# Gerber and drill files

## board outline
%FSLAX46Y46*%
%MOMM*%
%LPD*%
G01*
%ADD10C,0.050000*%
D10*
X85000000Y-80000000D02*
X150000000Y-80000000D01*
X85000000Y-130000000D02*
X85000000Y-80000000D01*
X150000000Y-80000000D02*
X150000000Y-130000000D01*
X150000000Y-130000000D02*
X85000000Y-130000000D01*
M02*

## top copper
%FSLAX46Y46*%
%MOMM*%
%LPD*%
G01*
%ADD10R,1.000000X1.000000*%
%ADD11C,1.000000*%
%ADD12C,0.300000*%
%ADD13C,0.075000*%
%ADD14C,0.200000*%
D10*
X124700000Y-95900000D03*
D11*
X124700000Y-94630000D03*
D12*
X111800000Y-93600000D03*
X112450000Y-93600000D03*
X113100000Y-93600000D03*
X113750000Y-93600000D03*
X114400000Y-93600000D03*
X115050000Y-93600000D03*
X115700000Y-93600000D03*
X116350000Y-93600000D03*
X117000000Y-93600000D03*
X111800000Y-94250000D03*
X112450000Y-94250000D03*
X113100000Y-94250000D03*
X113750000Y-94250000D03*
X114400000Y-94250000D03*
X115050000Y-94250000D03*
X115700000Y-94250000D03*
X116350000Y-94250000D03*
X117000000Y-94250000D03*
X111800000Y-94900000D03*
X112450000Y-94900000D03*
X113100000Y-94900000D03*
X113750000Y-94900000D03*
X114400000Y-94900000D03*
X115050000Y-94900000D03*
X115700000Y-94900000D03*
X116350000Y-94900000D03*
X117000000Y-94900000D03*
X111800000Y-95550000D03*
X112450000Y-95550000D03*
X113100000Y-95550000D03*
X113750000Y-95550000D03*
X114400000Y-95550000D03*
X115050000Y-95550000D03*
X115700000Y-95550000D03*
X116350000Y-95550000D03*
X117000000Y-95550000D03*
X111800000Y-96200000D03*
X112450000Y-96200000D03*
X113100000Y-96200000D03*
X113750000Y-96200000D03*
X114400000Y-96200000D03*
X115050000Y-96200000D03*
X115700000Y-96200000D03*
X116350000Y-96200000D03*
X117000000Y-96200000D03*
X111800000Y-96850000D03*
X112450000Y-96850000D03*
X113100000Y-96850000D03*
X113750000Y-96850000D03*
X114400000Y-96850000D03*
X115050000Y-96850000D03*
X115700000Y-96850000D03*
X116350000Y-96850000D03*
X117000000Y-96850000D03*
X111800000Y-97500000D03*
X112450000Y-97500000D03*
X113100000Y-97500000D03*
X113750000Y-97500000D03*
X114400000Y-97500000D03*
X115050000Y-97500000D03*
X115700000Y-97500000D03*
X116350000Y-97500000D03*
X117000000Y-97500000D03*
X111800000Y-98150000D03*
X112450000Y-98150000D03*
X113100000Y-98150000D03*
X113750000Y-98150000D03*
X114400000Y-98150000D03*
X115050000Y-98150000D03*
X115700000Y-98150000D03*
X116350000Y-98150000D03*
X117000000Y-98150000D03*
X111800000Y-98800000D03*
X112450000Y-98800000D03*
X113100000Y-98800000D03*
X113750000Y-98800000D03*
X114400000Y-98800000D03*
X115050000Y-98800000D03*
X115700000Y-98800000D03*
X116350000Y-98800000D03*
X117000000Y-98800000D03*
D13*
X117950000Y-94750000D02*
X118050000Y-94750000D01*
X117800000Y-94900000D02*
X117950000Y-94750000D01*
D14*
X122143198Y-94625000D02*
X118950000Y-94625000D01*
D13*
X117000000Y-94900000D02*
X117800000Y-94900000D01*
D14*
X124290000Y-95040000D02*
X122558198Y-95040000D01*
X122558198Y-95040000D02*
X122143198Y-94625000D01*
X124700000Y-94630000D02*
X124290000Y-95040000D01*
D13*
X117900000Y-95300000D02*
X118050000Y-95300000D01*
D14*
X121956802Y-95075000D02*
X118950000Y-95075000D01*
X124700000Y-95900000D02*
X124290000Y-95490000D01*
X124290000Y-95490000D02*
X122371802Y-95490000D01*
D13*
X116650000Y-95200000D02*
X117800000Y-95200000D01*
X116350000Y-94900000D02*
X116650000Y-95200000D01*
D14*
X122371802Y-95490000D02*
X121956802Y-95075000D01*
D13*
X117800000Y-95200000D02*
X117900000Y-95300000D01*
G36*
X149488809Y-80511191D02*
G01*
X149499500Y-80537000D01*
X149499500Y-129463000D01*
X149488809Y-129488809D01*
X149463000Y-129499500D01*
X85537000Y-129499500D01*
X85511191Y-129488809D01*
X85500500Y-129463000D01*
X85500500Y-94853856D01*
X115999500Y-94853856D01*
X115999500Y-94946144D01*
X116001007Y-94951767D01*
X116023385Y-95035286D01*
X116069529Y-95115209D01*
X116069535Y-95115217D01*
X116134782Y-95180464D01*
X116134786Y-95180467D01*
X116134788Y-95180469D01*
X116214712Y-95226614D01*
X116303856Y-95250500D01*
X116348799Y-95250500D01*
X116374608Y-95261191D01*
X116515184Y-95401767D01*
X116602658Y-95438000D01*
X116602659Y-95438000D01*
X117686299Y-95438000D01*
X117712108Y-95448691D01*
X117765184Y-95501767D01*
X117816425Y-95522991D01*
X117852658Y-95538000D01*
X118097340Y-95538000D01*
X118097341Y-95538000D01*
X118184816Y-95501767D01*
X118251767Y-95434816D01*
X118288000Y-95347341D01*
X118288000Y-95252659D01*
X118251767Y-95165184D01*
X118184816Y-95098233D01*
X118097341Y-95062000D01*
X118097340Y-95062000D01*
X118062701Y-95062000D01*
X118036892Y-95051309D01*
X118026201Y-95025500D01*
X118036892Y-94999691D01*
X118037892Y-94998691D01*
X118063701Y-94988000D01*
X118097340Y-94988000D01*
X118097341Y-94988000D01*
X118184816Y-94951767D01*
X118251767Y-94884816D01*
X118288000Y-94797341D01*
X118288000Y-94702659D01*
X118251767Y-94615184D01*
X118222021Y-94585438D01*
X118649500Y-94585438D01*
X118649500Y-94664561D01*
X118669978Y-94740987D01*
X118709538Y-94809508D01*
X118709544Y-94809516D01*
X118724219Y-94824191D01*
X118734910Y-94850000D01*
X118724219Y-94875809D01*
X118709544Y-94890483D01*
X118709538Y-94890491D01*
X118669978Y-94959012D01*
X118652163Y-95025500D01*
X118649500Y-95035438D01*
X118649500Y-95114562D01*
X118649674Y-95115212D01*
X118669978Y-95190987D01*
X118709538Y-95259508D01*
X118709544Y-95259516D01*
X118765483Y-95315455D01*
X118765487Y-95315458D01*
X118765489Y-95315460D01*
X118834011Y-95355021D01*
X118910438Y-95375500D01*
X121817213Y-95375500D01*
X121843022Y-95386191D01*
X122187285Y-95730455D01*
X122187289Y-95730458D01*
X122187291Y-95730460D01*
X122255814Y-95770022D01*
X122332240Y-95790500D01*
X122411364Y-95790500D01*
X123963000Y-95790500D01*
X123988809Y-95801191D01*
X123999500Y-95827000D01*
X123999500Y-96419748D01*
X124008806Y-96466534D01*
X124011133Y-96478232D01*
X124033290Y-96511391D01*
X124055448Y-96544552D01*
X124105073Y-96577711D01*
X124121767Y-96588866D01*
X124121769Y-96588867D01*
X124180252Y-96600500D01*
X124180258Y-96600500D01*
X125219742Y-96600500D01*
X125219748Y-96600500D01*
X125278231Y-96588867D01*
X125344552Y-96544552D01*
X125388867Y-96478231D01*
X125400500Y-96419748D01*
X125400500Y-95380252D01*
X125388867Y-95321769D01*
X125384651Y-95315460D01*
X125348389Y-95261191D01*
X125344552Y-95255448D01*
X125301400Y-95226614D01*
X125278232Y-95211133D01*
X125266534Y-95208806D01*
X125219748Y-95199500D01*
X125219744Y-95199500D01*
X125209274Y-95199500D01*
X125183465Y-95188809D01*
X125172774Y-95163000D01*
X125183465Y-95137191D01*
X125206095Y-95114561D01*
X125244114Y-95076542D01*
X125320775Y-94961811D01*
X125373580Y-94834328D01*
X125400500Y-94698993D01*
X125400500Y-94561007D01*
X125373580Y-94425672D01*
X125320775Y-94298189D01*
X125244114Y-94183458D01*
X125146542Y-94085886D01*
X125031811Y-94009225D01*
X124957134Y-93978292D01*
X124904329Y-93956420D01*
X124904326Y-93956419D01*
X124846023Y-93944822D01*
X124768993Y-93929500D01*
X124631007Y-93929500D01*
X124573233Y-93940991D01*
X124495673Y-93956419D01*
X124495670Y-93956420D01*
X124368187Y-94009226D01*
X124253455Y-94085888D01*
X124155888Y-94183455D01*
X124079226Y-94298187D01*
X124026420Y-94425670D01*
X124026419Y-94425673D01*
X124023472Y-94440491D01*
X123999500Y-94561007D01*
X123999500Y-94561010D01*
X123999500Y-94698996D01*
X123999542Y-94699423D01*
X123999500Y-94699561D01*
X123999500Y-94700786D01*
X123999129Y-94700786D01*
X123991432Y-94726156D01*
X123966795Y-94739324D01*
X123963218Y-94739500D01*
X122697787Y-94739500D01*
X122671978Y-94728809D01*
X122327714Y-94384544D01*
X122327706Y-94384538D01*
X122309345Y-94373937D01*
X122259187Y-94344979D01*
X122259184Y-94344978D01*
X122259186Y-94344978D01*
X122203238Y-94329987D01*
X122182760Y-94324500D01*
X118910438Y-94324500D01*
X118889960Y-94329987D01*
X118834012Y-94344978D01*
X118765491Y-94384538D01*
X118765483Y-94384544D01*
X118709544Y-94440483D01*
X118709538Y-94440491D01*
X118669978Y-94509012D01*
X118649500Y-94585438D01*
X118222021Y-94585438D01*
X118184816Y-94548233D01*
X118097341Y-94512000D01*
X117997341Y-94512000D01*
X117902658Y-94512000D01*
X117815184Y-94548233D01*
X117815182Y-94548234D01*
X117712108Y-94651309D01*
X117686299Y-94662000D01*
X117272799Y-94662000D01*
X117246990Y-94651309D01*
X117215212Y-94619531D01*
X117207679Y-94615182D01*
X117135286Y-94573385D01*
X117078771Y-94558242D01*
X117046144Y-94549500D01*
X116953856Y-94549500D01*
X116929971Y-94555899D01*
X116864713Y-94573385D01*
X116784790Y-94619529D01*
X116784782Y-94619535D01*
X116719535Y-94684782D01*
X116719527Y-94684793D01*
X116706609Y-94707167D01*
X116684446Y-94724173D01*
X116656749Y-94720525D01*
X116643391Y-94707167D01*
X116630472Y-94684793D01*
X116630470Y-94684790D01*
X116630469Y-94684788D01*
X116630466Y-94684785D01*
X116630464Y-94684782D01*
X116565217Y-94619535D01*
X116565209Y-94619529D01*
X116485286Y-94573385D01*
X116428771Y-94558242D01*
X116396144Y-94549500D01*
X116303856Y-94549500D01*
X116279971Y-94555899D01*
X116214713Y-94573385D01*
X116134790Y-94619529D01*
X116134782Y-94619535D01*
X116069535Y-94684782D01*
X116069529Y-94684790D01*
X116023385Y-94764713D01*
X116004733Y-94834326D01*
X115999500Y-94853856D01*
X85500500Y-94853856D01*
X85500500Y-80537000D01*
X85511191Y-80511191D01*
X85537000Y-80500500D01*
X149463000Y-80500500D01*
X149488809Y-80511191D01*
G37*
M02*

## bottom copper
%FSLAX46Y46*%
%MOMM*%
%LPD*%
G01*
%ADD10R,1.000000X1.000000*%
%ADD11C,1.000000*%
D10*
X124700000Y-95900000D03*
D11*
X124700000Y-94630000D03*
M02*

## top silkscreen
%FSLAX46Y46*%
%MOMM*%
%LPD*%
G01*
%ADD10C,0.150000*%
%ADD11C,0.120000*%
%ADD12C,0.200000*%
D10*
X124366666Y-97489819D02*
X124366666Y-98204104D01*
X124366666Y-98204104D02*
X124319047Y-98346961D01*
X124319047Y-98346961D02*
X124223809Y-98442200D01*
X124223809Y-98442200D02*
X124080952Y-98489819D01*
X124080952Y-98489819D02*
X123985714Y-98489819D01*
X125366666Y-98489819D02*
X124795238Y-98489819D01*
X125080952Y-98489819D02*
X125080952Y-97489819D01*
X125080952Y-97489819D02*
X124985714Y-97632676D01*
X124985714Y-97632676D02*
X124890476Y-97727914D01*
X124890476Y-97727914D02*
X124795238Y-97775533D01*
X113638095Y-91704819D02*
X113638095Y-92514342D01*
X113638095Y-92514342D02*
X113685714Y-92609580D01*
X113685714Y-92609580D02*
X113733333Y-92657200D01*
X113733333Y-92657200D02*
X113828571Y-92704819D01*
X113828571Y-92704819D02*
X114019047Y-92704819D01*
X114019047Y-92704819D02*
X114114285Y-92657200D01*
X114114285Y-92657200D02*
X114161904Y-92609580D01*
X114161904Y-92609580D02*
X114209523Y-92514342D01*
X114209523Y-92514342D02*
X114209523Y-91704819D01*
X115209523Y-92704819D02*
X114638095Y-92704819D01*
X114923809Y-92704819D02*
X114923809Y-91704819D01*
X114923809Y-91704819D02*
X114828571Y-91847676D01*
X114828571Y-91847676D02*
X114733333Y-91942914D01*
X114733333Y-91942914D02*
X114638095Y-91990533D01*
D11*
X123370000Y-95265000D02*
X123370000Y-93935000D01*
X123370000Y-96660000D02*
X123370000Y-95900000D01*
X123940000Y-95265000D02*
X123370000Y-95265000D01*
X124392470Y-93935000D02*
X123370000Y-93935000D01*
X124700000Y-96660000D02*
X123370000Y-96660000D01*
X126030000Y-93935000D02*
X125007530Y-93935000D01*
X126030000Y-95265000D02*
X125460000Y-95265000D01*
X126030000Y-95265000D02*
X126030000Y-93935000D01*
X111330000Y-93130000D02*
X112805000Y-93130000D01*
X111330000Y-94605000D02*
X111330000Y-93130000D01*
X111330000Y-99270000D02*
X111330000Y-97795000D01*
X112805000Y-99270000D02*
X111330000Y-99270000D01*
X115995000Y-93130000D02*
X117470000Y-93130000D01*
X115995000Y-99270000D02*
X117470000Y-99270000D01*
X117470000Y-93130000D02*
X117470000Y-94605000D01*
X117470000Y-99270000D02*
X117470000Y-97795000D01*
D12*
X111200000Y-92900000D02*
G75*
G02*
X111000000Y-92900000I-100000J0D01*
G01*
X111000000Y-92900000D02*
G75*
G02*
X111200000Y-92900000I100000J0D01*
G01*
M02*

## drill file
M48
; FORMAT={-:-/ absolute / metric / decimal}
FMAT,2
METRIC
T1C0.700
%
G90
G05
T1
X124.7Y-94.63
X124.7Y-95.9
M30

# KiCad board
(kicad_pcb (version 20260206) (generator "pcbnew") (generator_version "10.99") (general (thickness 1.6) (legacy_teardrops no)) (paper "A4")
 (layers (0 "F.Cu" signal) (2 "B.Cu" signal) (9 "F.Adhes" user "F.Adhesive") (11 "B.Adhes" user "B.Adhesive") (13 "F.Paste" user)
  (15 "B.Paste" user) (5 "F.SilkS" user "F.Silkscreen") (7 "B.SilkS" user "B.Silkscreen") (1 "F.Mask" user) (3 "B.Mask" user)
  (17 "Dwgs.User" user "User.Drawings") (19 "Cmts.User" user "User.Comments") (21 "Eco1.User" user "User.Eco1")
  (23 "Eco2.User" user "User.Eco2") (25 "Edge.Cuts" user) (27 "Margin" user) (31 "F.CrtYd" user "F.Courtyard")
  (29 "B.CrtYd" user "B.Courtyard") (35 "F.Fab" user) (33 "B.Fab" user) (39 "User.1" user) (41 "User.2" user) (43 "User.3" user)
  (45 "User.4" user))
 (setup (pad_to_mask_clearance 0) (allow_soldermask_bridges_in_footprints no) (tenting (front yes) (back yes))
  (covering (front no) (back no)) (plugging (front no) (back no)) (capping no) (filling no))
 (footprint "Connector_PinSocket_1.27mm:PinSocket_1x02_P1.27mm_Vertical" (layer "F.Cu") (at 124.7 95.9 180)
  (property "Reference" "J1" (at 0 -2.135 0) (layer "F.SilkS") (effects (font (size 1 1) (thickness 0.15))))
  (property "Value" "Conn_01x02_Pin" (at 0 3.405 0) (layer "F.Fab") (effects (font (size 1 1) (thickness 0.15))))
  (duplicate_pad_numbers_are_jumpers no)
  (fp_line (start 1.33 0.635) (end 1.33 1.965) (stroke (width 0.12) (type solid)) (layer "F.SilkS"))
  (fp_line (start 1.33 -0.76) (end 1.33 0) (stroke (width 0.12) (type solid)) (layer "F.SilkS"))
  (fp_line (start 0.76 0.635) (end 1.33 0.635) (stroke (width 0.12) (type solid)) (layer "F.SilkS"))
  (fp_line (start 0.30753 1.965) (end 1.33 1.965) (stroke (width 0.12) (type solid)) (layer "F.SilkS"))
  (fp_line (start 0 -0.76) (end 1.33 -0.76) (stroke (width 0.12) (type solid)) (layer "F.SilkS"))
  (fp_line (start -1.33 1.965) (end -0.30753 1.965) (stroke (width 0.12) (type solid)) (layer "F.SilkS"))
  (fp_line (start -1.33 0.635) (end -0.76 0.635) (stroke (width 0.12) (type solid)) (layer "F.SilkS"))
  (fp_line (start -1.33 0.635) (end -1.33 1.965) (stroke (width 0.12) (type solid)) (layer "F.SilkS"))
  (pad "1" thru_hole rect (at 0 0 180) (size 1 1) (drill 0.7) (layers "*.Cu" "*.Mask") (remove_unused_layers no) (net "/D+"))
  (pad "2" thru_hole circle (at 0 1.27 180) (size 1 1) (drill 0.7) (layers "*.Cu" "*.Mask") (remove_unused_layers no) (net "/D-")))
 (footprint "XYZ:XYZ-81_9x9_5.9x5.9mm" (layer "F.Cu") (at 114.4 96.2)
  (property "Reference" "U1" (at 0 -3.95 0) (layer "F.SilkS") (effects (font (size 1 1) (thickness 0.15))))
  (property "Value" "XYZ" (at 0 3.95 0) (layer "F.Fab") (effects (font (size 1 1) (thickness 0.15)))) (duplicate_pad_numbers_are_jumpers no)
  (fp_line (start -3.07 -3.07) (end -1.595 -3.07) (stroke (width 0.12) (type default)) (layer "F.SilkS"))
  (fp_line (start -3.07 -1.595) (end -3.07 -3.07) (stroke (width 0.12) (type default)) (layer "F.SilkS"))
  (fp_line (start -3.07 3.07) (end -3.07 1.595) (stroke (width 0.12) (type default)) (layer "F.SilkS"))
  (fp_line (start -1.595 3.07) (end -3.07 3.07) (stroke (width 0.12) (type default)) (layer "F.SilkS"))
  (fp_line (start 1.595 -3.07) (end 3.07 -3.07) (stroke (width 0.12) (type default)) (layer "F.SilkS"))
  (fp_line (start 1.595 3.07) (end 3.07 3.07) (stroke (width 0.12) (type default)) (layer "F.SilkS"))
  (fp_line (start 3.07 -3.07) (end 3.07 -1.595) (stroke (width 0.12) (type default)) (layer "F.SilkS"))
  (fp_line (start 3.07 3.07) (end 3.07 1.595) (stroke (width 0.12) (type default)) (layer "F.SilkS"))
  (fp_circle (center -3.3 -3.3) (end -3.3 -3.2) (stroke (width 0.2) (type default)) (fill no) (layer "F.SilkS"))
  (pad "A1" smd circle (at -2.6 -2.6) (size 0.3 0.3) (layers "F.Cu" "F.Mask" "F.Paste") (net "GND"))
  (pad "A2" smd circle (at -1.95 -2.6) (size 0.3 0.3) (layers "F.Cu" "F.Mask" "F.Paste") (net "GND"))
  (pad "A3" smd circle (at -1.3 -2.6) (size 0.3 0.3) (layers "F.Cu" "F.Mask" "F.Paste") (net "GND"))
  (pad "A4" smd circle (at -0.65 -2.6) (size 0.3 0.3) (layers "F.Cu" "F.Mask" "F.Paste") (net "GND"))
  (pad "A5" smd circle (at 0 -2.6) (size 0.3 0.3) (layers "F.Cu" "F.Mask" "F.Paste") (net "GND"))
  (pad "A6" smd circle (at 0.65 -2.6) (size 0.3 0.3) (layers "F.Cu" "F.Mask" "F.Paste") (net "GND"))
  (pad "A7" smd circle (at 1.3 -2.6) (size 0.3 0.3) (layers "F.Cu" "F.Mask" "F.Paste") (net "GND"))
  (pad "A8" smd circle (at 1.95 -2.6) (size 0.3 0.3) (layers "F.Cu" "F.Mask" "F.Paste") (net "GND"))
  (pad "A9" smd circle (at 2.6 -2.6) (size 0.3 0.3) (layers "F.Cu" "F.Mask" "F.Paste") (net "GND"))
  (pad "B1" smd circle (at -2.6 -1.95) (size 0.3 0.3) (layers "F.Cu" "F.Mask" "F.Paste") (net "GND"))
  (pad "B2" smd circle (at -1.95 -1.95) (size 0.3 0.3) (layers "F.Cu" "F.Mask" "F.Paste") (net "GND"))
  (pad "B3" smd circle (at -1.3 -1.95) (size 0.3 0.3) (layers "F.Cu" "F.Mask" "F.Paste") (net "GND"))
  (pad "B4" smd circle (at -0.65 -1.95) (size 0.3 0.3) (layers "F.Cu" "F.Mask" "F.Paste") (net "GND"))
  (pad "B5" smd circle (at 0 -1.95) (size 0.3 0.3) (layers "F.Cu" "F.Mask" "F.Paste") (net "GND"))
  (pad "B6" smd circle (at 0.65 -1.95) (size 0.3 0.3) (layers "F.Cu" "F.Mask" "F.Paste") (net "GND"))
  (pad "B7" smd circle (at 1.3 -1.95) (size 0.3 0.3) (layers "F.Cu" "F.Mask" "F.Paste") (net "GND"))
  (pad "B8" smd circle (at 1.95 -1.95) (size 0.3 0.3) (layers "F.Cu" "F.Mask" "F.Paste") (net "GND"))
  (pad "B9" smd circle (at 2.6 -1.95) (size 0.3 0.3) (layers "F.Cu" "F.Mask" "F.Paste") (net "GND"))
  (pad "C1" smd circle (at -2.6 -1.3) (size 0.3 0.3) (layers "F.Cu" "F.Mask" "F.Paste") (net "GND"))
  (pad "C2" smd circle (at -1.95 -1.3) (size 0.3 0.3) (layers "F.Cu" "F.Mask" "F.Paste") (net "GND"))
  (pad "C3" smd circle (at -1.3 -1.3) (size 0.3 0.3) (layers "F.Cu" "F.Mask" "F.Paste") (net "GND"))
  (pad "C4" smd circle (at -0.65 -1.3) (size 0.3 0.3) (layers "F.Cu" "F.Mask" "F.Paste") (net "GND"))
  (pad "C5" smd circle (at 0 -1.3) (size 0.3 0.3) (layers "F.Cu" "F.Mask" "F.Paste") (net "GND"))
  (pad "C6" smd circle (at 0.65 -1.3) (size 0.3 0.3) (layers "F.Cu" "F.Mask" "F.Paste") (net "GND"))
  (pad "C7" smd circle (at 1.3 -1.3) (size 0.3 0.3) (layers "F.Cu" "F.Mask" "F.Paste") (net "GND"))
  (pad "C8" smd circle (at 1.95 -1.3) (size 0.3 0.3) (layers "F.Cu" "F.Mask" "F.Paste") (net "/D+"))
  (pad "C9" smd circle (at 2.6 -1.3) (size 0.3 0.3) (layers "F.Cu" "F.Mask" "F.Paste") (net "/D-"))
  (pad "D1" smd circle (at -2.6 -0.65) (size 0.3 0.3) (layers "F.Cu" "F.Mask" "F.Paste") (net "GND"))
  (pad "D2" smd circle (at -1.95 -0.65) (size 0.3 0.3) (layers "F.Cu" "F.Mask" "F.Paste") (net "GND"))
  (pad "D3" smd circle (at -1.3 -0.65) (size 0.3 0.3) (layers "F.Cu" "F.Mask" "F.Paste") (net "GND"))
  (pad "D4" smd circle (at -0.65 -0.65) (size 0.3 0.3) (layers "F.Cu" "F.Mask" "F.Paste") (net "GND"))
  (pad "D5" smd circle (at 0 -0.65) (size 0.3 0.3) (layers "F.Cu" "F.Mask" "F.Paste") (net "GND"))
  (pad "D6" smd circle (at 0.65 -0.65) (size 0.3 0.3) (layers "F.Cu" "F.Mask" "F.Paste") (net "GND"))
  (pad "D7" smd circle (at 1.3 -0.65) (size 0.3 0.3) (layers "F.Cu" "F.Mask" "F.Paste") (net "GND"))
  (pad "D8" smd circle (at 1.95 -0.65) (size 0.3 0.3) (layers "F.Cu" "F.Mask" "F.Paste") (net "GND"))
  (pad "D9" smd circle (at 2.6 -0.65) (size 0.3 0.3) (layers "F.Cu" "F.Mask" "F.Paste") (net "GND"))
  (pad "E1" smd circle (at -2.6 0) (size 0.3 0.3) (layers "F.Cu" "F.Mask" "F.Paste") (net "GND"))
  (pad "E2" smd circle (at -1.95 0) (size 0.3 0.3) (layers "F.Cu" "F.Mask" "F.Paste") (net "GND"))
  (pad "E3" smd circle (at -1.3 0) (size 0.3 0.3) (layers "F.Cu" "F.Mask" "F.Paste") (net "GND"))
  (pad "E4" smd circle (at -0.65 0) (size 0.3 0.3) (layers "F.Cu" "F.Mask" "F.Paste") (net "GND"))
  (pad "E5" smd circle (at 0 0) (size 0.3 0.3) (layers "F.Cu" "F.Mask" "F.Paste") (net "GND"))
  (pad "E6" smd circle (at 0.65 0) (size 0.3 0.3) (layers "F.Cu" "F.Mask" "F.Paste") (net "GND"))
  (pad "E7" smd circle (at 1.3 0) (size 0.3 0.3) (layers "F.Cu" "F.Mask" "F.Paste") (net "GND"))
  (pad "E8" smd circle (at 1.95 0) (size 0.3 0.3) (layers "F.Cu" "F.Mask" "F.Paste") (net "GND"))
  (pad "E9" smd circle (at 2.6 0) (size 0.3 0.3) (layers "F.Cu" "F.Mask" "F.Paste") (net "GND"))
  (pad "F1" smd circle (at -2.6 0.65) (size 0.3 0.3) (layers "F.Cu" "F.Mask" "F.Paste") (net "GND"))
  (pad "F2" smd circle (at -1.95 0.65) (size 0.3 0.3) (layers "F.Cu" "F.Mask" "F.Paste") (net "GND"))
  (pad "F3" smd circle (at -1.3 0.65) (size 0.3 0.3) (layers "F.Cu" "F.Mask" "F.Paste") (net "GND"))
  (pad "F4" smd circle (at -0.65 0.65) (size 0.3 0.3) (layers "F.Cu" "F.Mask" "F.Paste") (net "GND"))
  (pad "F5" smd circle (at 0 0.65) (size 0.3 0.3) (layers "F.Cu" "F.Mask" "F.Paste") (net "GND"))
  (pad "F6" smd circle (at 0.65 0.65) (size 0.3 0.3) (layers "F.Cu" "F.Mask" "F.Paste") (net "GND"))
  (pad "F7" smd circle (at 1.3 0.65) (size 0.3 0.3) (layers "F.Cu" "F.Mask" "F.Paste") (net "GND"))
  (pad "F8" smd circle (at 1.95 0.65) (size 0.3 0.3) (layers "F.Cu" "F.Mask" "F.Paste") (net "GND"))
  (pad "F9" smd circle (at 2.6 0.65) (size 0.3 0.3) (layers "F.Cu" "F.Mask" "F.Paste") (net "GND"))
  (pad "G1" smd circle (at -2.6 1.3) (size 0.3 0.3) (layers "F.Cu" "F.Mask" "F.Paste") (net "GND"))
  (pad "G2" smd circle (at -1.95 1.3) (size 0.3 0.3) (layers "F.Cu" "F.Mask" "F.Paste") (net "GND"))
  (pad "G3" smd circle (at -1.3 1.3) (size 0.3 0.3) (layers "F.Cu" "F.Mask" "F.Paste") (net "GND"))
  (pad "G4" smd circle (at -0.65 1.3) (size 0.3 0.3) (layers "F.Cu" "F.Mask" "F.Paste") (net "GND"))
  (pad "G5" smd circle (at 0 1.3) (size 0.3 0.3) (layers "F.Cu" "F.Mask" "F.Paste") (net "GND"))
  (pad "G6" smd circle (at 0.65 1.3) (size 0.3 0.3) (layers "F.Cu" "F.Mask" "F.Paste") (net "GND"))
  (pad "G7" smd circle (at 1.3 1.3) (size 0.3 0.3) (layers "F.Cu" "F.Mask" "F.Paste") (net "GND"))
  (pad "G8" smd circle (at 1.95 1.3) (size 0.3 0.3) (layers "F.Cu" "F.Mask" "F.Paste") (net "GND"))
  (pad "G9" smd circle (at 2.6 1.3) (size 0.3 0.3) (layers "F.Cu" "F.Mask" "F.Paste") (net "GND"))
  (pad "H1" smd circle (at -2.6 1.95) (size 0.3 0.3) (layers "F.Cu" "F.Mask" "F.Paste") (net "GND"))
  (pad "H2" smd circle (at -1.95 1.95) (size 0.3 0.3) (layers "F.Cu" "F.Mask" "F.Paste") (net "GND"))
  (pad "H3" smd circle (at -1.3 1.95) (size 0.3 0.3) (layers "F.Cu" "F.Mask" "F.Paste") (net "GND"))
  (pad "H4" smd circle (at -0.65 1.95) (size 0.3 0.3) (layers "F.Cu" "F.Mask" "F.Paste") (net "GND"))
  (pad "H5" smd circle (at 0 1.95) (size 0.3 0.3) (layers "F.Cu" "F.Mask" "F.Paste") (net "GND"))
  (pad "H6" smd circle (at 0.65 1.95) (size 0.3 0.3) (layers "F.Cu" "F.Mask" "F.Paste") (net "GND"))
  (pad "H7" smd circle (at 1.3 1.95) (size 0.3 0.3) (layers "F.Cu" "F.Mask" "F.Paste") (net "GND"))
  (pad "H8" smd circle (at 1.95 1.95) (size 0.3 0.3) (layers "F.Cu" "F.Mask" "F.Paste") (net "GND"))
  (pad "H9" smd circle (at 2.6 1.95) (size 0.3 0.3) (layers "F.Cu" "F.Mask" "F.Paste") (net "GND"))
  (pad "J1" smd circle (at -2.6 2.6) (size 0.3 0.3) (layers "F.Cu" "F.Mask" "F.Paste") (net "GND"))
  (pad "J2" smd circle (at -1.95 2.6) (size 0.3 0.3) (layers "F.Cu" "F.Mask" "F.Paste") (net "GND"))
  (pad "J3" smd circle (at -1.3 2.6) (size 0.3 0.3) (layers "F.Cu" "F.Mask" "F.Paste") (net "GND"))
  (pad "J4" smd circle (at -0.65 2.6) (size 0.3 0.3) (layers "F.Cu" "F.Mask" "F.Paste") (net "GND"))
  (pad "J5" smd circle (at 0 2.6) (size 0.3 0.3) (layers "F.Cu" "F.Mask" "F.Paste") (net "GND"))
  (pad "J6" smd circle (at 0.65 2.6) (size 0.3 0.3) (layers "F.Cu" "F.Mask" "F.Paste") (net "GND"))
  (pad "J7" smd circle (at 1.3 2.6) (size 0.3 0.3) (layers "F.Cu" "F.Mask" "F.Paste") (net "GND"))
  (pad "J8" smd circle (at 1.95 2.6) (size 0.3 0.3) (layers "F.Cu" "F.Mask" "F.Paste") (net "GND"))
  (pad "J9" smd circle (at 2.6 2.6) (size 0.3 0.3) (layers "F.Cu" "F.Mask" "F.Paste") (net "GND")))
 (gr_line (start 85 80) (end 150 80) (stroke (width 0.05) (type default)) (layer "Edge.Cuts"))
 (gr_line (start 85 130) (end 85 80) (stroke (width 0.05) (type default)) (layer "Edge.Cuts"))
 (gr_line (start 150 80) (end 150 130) (stroke (width 0.05) (type default)) (layer "Edge.Cuts"))
 (gr_line (start 150 130) (end 85 130) (stroke (width 0.05) (type default)) (layer "Edge.Cuts"))
 (segment (start 117.95 94.75) (end 118.05 94.75) (width 0.075) (layer "F.Cu") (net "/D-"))
 (segment (start 117.8 94.9) (end 117.95 94.75) (width 0.075) (layer "F.Cu") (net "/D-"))
 (segment (start 122.143198 94.625) (end 118.95 94.625) (width 0.2) (layer "F.Cu") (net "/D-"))
 (segment (start 117 94.9) (end 117.8 94.9) (width 0.075) (layer "F.Cu") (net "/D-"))
 (segment (start 124.29 95.04) (end 122.558198 95.04) (width 0.2) (layer "F.Cu") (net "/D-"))
 (segment (start 122.558198 95.04) (end 122.143198 94.625) (width 0.2) (layer "F.Cu") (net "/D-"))
 (segment (start 124.7 94.63) (end 124.29 95.04) (width 0.2) (layer "F.Cu") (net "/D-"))
 (segment (start 117.9 95.3) (end 118.05 95.3) (width 0.075) (layer "F.Cu") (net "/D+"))
 (segment (start 121.956802 95.075) (end 118.95 95.075) (width 0.2) (layer "F.Cu") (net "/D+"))
 (segment (start 124.7 95.9) (end 124.29 95.49) (width 0.2) (layer "F.Cu") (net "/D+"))
 (segment (start 124.29 95.49) (end 122.371802 95.49) (width 0.2) (layer "F.Cu") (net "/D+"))
 (segment (start 116.65 95.2) (end 117.8 95.2) (width 0.075) (layer "F.Cu") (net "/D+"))
 (segment (start 116.35 94.9) (end 116.65 95.2) (width 0.075) (layer "F.Cu") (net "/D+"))
 (segment (start 122.371802 95.49) (end 121.956802 95.075) (width 0.2) (layer "F.Cu") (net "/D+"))
 (segment (start 117.8 95.2) (end 117.9 95.3) (width 0.075) (layer "F.Cu") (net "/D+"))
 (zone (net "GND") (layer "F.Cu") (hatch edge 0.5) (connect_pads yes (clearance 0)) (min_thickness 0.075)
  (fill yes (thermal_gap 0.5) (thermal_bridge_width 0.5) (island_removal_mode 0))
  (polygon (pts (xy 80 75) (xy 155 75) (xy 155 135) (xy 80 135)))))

